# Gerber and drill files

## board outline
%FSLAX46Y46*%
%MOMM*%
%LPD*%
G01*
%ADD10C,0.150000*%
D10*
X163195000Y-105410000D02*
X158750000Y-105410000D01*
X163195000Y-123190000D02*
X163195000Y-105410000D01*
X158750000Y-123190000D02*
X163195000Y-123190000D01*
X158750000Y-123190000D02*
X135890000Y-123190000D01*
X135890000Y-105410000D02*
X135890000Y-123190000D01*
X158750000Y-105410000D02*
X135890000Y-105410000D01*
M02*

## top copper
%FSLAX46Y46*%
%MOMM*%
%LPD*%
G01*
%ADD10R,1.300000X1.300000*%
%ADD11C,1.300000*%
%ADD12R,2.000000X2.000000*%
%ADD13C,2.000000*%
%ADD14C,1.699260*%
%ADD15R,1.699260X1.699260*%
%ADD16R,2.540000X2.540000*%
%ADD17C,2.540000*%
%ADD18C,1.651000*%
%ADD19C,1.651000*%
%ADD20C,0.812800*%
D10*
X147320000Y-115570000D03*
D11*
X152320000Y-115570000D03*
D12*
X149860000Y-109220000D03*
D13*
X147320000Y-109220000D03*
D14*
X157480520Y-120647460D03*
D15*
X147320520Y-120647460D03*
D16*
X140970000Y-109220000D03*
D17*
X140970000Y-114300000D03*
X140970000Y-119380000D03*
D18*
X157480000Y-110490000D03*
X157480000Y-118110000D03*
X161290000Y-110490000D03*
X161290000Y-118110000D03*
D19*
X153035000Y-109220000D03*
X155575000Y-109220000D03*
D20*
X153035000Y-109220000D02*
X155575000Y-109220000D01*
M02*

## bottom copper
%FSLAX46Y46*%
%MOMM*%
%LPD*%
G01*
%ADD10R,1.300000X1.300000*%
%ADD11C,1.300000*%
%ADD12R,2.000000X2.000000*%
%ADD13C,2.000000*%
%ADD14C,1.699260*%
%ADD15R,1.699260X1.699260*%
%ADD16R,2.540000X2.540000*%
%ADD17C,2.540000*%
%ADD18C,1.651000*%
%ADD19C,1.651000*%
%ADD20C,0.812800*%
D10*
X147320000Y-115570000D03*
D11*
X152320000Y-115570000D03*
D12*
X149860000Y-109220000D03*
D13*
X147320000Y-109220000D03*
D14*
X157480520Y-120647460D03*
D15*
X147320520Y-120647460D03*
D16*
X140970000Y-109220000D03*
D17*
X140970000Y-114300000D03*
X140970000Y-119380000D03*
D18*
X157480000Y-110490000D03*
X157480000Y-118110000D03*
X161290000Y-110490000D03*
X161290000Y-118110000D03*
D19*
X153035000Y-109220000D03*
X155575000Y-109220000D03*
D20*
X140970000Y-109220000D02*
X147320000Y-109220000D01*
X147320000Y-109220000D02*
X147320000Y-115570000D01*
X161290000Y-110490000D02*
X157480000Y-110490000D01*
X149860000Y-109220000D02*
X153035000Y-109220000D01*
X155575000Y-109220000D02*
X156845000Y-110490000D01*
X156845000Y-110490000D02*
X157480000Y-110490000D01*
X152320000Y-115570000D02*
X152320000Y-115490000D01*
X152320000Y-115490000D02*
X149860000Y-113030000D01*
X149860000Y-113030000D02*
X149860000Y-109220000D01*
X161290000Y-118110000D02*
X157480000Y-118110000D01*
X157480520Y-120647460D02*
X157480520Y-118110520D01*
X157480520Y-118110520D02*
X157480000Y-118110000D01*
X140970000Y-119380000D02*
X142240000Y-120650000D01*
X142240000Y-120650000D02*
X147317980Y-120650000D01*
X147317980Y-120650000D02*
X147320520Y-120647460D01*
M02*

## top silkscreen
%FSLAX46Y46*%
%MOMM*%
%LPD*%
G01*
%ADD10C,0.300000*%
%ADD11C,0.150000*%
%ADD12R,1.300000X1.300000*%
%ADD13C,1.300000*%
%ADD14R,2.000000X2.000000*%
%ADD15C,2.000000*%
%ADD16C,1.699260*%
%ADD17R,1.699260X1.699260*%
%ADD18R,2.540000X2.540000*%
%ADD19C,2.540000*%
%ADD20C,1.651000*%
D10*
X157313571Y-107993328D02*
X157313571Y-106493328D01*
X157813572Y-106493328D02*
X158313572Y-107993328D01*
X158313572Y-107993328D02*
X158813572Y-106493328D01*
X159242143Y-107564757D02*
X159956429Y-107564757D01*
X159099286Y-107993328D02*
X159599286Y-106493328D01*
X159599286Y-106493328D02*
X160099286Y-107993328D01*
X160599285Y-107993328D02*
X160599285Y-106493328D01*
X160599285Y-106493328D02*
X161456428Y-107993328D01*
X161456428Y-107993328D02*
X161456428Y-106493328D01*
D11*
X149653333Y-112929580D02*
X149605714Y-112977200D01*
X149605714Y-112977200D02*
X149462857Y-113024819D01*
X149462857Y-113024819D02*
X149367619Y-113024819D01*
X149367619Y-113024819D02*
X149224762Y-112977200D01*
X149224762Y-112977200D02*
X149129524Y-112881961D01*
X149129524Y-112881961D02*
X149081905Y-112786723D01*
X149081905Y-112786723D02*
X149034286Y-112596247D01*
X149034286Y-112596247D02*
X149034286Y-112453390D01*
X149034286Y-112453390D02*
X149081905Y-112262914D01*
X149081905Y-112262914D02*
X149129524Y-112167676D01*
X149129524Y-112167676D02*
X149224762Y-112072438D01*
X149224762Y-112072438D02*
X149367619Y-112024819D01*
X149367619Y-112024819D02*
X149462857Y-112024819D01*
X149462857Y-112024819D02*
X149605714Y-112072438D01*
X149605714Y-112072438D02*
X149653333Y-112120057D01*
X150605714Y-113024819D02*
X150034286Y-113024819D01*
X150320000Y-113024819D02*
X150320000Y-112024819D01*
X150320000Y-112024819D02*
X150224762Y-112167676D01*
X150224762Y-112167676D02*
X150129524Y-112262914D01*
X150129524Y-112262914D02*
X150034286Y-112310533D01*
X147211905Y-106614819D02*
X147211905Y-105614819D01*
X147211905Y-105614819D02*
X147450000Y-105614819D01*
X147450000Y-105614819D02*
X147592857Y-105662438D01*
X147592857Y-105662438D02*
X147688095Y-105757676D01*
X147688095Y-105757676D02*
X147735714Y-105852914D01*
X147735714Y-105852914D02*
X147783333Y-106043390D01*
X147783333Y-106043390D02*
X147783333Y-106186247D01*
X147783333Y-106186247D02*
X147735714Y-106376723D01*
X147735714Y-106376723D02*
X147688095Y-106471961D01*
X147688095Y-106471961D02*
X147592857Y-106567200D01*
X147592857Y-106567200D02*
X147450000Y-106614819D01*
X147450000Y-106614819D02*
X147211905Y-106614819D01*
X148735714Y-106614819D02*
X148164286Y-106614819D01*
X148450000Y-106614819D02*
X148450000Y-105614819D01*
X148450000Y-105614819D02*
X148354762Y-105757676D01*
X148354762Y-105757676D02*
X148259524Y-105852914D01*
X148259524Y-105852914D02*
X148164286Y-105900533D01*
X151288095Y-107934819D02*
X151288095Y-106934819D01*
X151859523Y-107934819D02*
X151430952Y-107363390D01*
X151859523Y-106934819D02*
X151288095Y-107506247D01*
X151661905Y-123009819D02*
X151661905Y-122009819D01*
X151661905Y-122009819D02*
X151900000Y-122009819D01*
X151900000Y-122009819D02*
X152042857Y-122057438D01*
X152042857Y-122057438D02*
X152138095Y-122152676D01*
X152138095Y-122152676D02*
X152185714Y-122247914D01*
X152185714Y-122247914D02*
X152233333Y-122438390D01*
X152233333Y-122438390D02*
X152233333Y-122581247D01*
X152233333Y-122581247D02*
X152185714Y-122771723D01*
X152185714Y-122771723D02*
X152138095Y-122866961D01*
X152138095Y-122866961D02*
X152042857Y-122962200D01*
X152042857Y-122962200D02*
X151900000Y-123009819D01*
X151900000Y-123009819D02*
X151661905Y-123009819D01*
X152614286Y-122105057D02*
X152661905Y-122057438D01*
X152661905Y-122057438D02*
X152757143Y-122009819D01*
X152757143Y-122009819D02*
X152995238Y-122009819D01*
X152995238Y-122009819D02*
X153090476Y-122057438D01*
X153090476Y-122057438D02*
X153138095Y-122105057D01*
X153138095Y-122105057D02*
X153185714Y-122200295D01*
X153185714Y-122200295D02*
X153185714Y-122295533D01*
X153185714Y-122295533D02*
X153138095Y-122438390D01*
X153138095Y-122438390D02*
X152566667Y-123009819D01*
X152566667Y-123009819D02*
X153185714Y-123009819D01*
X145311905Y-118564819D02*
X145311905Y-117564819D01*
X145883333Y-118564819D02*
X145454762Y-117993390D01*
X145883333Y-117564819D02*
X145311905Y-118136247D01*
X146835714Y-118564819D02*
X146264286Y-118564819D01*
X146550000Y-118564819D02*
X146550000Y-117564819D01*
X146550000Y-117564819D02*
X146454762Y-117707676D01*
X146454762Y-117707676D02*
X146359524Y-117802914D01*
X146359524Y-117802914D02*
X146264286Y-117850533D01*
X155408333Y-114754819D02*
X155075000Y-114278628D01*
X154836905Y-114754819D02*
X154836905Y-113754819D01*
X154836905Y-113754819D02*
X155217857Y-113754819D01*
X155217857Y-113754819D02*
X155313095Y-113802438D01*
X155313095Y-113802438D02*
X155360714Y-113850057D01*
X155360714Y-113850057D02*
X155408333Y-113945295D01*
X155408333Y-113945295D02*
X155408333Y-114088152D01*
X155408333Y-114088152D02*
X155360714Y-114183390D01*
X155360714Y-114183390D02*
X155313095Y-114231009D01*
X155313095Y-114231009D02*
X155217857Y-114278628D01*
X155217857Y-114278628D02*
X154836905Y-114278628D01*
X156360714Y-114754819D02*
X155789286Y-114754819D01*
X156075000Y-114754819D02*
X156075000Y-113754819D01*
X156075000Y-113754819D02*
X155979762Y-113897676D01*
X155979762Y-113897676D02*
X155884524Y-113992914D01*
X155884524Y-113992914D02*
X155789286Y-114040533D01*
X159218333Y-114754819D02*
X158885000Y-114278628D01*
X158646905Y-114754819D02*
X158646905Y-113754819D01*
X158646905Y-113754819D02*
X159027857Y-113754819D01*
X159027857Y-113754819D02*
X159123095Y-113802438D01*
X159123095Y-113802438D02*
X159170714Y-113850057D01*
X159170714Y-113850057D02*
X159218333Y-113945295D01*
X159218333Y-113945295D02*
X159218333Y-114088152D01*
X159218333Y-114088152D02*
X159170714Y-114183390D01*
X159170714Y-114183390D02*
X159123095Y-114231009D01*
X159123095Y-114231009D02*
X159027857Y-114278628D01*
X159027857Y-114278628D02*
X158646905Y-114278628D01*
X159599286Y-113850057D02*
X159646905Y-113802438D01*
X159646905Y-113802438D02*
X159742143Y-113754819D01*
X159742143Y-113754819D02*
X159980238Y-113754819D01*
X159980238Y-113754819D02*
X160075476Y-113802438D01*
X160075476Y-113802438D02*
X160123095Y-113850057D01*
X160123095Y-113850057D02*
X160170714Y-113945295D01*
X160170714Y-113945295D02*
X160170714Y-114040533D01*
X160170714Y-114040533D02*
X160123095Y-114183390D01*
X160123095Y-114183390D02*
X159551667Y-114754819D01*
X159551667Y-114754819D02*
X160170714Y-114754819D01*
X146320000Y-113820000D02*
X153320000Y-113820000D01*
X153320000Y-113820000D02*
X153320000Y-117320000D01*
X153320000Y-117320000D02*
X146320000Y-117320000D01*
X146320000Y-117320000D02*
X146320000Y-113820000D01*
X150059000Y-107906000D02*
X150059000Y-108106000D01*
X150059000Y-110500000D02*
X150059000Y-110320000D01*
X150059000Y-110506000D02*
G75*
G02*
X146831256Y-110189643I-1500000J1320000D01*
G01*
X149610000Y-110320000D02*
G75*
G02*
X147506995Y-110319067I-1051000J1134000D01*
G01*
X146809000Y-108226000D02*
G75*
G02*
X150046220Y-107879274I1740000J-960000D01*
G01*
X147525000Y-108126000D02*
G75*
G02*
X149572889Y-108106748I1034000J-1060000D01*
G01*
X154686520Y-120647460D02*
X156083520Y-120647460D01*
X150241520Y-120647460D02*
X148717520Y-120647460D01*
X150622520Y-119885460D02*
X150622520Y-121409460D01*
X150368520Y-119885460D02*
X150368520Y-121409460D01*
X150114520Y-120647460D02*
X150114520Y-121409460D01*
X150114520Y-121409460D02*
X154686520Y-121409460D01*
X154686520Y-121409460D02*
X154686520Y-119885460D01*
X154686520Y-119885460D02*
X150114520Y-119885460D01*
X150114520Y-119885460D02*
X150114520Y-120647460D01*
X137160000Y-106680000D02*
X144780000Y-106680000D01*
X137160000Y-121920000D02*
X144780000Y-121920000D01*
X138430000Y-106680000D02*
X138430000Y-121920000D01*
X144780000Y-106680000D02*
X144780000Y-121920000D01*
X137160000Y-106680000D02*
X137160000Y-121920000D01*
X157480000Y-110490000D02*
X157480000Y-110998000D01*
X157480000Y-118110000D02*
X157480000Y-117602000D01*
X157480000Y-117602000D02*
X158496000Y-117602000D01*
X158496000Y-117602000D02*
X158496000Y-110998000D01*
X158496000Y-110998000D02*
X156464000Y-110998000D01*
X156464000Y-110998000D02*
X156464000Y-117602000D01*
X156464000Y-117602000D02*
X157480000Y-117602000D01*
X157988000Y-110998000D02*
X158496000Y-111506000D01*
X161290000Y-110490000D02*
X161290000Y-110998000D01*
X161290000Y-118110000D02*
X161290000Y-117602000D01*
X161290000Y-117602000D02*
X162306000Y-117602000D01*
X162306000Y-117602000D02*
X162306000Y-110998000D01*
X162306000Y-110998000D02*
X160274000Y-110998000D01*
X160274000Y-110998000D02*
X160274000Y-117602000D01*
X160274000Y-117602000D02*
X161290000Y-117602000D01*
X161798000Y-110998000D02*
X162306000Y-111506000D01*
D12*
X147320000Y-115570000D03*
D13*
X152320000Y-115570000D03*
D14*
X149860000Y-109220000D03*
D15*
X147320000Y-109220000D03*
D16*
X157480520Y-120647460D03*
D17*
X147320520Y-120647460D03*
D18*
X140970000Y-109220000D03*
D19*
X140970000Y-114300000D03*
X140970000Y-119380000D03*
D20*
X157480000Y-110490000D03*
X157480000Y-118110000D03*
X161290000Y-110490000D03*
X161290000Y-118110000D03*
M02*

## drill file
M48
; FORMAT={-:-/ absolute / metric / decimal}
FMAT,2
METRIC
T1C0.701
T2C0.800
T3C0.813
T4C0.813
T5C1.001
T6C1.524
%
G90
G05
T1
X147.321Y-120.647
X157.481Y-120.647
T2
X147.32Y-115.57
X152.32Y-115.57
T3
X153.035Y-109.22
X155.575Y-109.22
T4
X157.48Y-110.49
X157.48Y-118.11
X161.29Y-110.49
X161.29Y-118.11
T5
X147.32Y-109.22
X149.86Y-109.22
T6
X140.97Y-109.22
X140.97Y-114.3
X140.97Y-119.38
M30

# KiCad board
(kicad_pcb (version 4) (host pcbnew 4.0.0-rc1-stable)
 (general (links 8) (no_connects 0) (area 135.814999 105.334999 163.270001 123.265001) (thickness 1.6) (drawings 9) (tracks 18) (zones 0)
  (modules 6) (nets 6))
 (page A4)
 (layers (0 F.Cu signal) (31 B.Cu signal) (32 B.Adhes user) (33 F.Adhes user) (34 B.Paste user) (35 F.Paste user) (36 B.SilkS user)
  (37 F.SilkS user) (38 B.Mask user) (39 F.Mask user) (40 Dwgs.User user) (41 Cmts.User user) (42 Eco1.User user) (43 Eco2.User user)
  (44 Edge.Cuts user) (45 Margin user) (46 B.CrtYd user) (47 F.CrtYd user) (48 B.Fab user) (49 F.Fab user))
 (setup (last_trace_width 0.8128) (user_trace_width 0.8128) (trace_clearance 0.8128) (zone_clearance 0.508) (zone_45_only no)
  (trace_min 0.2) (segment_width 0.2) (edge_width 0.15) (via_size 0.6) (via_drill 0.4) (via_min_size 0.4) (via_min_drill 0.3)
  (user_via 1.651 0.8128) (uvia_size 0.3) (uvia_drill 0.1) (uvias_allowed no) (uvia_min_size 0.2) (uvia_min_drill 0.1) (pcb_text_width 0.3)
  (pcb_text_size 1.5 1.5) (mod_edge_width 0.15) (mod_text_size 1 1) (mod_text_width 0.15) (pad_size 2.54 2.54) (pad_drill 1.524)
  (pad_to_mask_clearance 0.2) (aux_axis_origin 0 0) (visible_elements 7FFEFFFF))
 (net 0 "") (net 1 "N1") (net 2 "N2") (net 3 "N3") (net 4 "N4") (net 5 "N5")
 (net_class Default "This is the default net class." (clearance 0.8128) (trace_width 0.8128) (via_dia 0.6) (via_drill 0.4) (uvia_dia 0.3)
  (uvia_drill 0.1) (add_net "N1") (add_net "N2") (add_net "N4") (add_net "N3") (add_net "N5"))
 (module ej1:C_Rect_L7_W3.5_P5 (layer F.Cu) (at 147.32 115.57)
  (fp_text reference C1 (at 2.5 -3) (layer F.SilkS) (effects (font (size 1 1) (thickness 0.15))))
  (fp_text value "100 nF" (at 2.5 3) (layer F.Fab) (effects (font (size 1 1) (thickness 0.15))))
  (fp_line (start -1 -1.75) (end 6 -1.75) (layer F.SilkS) (width 0.15))
  (fp_line (start 6 -1.75) (end 6 1.75) (layer F.SilkS) (width 0.15))
  (fp_line (start 6 1.75) (end -1 1.75) (layer F.SilkS) (width 0.15))
  (fp_line (start -1 1.75) (end -1 -1.75) (layer F.SilkS) (width 0.15))
  (pad 1 thru_hole rect (at 0 0) (size 1.3 1.3) (drill 0.8) (layers *.Cu *.Mask F.SilkS) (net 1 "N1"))
  (pad 2 thru_hole circle (at 5 0) (size 1.3 1.3) (drill 0.8) (layers *.Cu *.Mask F.SilkS) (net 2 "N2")))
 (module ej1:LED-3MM (layer F.Cu) (at 149.86 109.22 180)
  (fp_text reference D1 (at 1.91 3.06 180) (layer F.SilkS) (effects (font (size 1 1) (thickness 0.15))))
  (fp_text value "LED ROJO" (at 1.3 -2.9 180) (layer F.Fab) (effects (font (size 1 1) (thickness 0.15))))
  (fp_line (start -0.199 1.314) (end -0.199 1.114) (layer F.SilkS) (width 0.15))
  (fp_line (start -0.199 -1.28) (end -0.199 -1.1) (layer F.SilkS) (width 0.15))
  (fp_arc (start 1.301 0.034) (end -0.199 -1.286) (angle 108.5) (layer F.SilkS) (width 0.15))
  (fp_arc (start 1.301 0.034) (end 0.25 -1.1) (angle 85.7) (layer F.SilkS) (width 0.15))
  (fp_arc (start 1.311 0.034) (end 3.051 0.994) (angle 110) (layer F.SilkS) (width 0.15))
  (fp_arc (start 1.301 0.034) (end 2.335 1.094) (angle 87.5) (layer F.SilkS) (width 0.15))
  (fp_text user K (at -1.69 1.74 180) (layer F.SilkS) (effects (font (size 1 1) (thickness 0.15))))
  (pad 1 thru_hole rect (at 0 0 270) (size 2 2) (drill 1.00076) (layers *.Cu *.Mask F.SilkS) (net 2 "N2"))
  (pad 2 thru_hole circle (at 2.54 0 180) (size 2 2) (drill 1.00076) (layers *.Cu *.Mask F.SilkS) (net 1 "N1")))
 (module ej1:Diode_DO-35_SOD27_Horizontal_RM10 (layer F.Cu) (at 147.32 120.65)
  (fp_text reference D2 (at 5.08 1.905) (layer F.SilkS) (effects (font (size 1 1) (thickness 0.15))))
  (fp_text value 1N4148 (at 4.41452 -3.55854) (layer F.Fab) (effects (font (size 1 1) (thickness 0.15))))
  (fp_line (start 7.36652 -0.00254) (end 8.76352 -0.00254) (layer F.SilkS) (width 0.15))
  (fp_line (start 2.92152 -0.00254) (end 1.39752 -0.00254) (layer F.SilkS) (width 0.15))
  (fp_line (start 3.30252 -0.76454) (end 3.30252 0.75946) (layer F.SilkS) (width 0.15))
  (fp_line (start 3.04852 -0.76454) (end 3.04852 0.75946) (layer F.SilkS) (width 0.15))
  (fp_line (start 2.79452 -0.00254) (end 2.79452 0.75946) (layer F.SilkS) (width 0.15))
  (fp_line (start 2.79452 0.75946) (end 7.36652 0.75946) (layer F.SilkS) (width 0.15))
  (fp_line (start 7.36652 0.75946) (end 7.36652 -0.76454) (layer F.SilkS) (width 0.15))
  (fp_line (start 7.36652 -0.76454) (end 2.79452 -0.76454) (layer F.SilkS) (width 0.15))
  (fp_line (start 2.79452 -0.76454) (end 2.79452 -0.00254) (layer F.SilkS) (width 0.15))
  (pad 2 thru_hole circle (at 10.16052 -0.00254 180) (size 1.69926 1.69926) (drill 0.70104) (layers *.Cu *.Mask F.SilkS) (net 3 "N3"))
  (pad 1 thru_hole rect (at 0.00052 -0.00254 180) (size 1.69926 1.69926) (drill 0.70104) (layers *.Cu *.Mask F.SilkS) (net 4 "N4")))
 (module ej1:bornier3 (layer F.Cu) (at 140.97 114.3 270)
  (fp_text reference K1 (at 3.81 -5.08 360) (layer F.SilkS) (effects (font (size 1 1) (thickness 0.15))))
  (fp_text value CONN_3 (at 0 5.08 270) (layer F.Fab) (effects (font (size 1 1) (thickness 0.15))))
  (fp_line (start -7.62 3.81) (end -7.62 -3.81) (layer F.SilkS) (width 0.15))
  (fp_line (start 7.62 3.81) (end 7.62 -3.81) (layer F.SilkS) (width 0.15))
  (fp_line (start -7.62 2.54) (end 7.62 2.54) (layer F.SilkS) (width 0.15))
  (fp_line (start -7.62 -3.81) (end 7.62 -3.81) (layer F.SilkS) (width 0.15))
  (fp_line (start -7.62 3.81) (end 7.62 3.81) (layer F.SilkS) (width 0.15))
  (pad 1 thru_hole rect (at -5.08 0 270) (size 2.54 2.54) (drill 1.524) (layers *.Cu *.Mask F.SilkS) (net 1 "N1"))
  (pad 2 thru_hole circle (at 0 0 270) (size 2.54 2.54) (drill 1.524) (layers *.Cu *.Mask F.SilkS) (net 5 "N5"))
  (pad 3 thru_hole circle (at 5.08 0 270) (size 2.54 2.54) (drill 1.524) (layers *.Cu *.Mask F.SilkS) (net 4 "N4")))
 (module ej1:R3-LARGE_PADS (layer F.Cu) (at 157.48 114.3 270)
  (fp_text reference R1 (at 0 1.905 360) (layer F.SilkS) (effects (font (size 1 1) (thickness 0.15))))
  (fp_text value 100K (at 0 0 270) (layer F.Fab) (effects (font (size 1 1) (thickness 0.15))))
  (fp_line (start -3.81 0) (end -3.302 0) (layer F.SilkS) (width 0.15))
  (fp_line (start 3.81 0) (end 3.302 0) (layer F.SilkS) (width 0.15))
  (fp_line (start 3.302 0) (end 3.302 -1.016) (layer F.SilkS) (width 0.15))
  (fp_line (start 3.302 -1.016) (end -3.302 -1.016) (layer F.SilkS) (width 0.15))
  (fp_line (start -3.302 -1.016) (end -3.302 1.016) (layer F.SilkS) (width 0.15))
  (fp_line (start -3.302 1.016) (end 3.302 1.016) (layer F.SilkS) (width 0.15))
  (fp_line (start 3.302 1.016) (end 3.302 0) (layer F.SilkS) (width 0.15))
  (fp_line (start -3.302 -0.508) (end -2.794 -1.016) (layer F.SilkS) (width 0.15))
  (pad 1 thru_hole circle (at -3.81 0 270) (size 1.651 1.651) (drill 0.8128) (layers *.Cu *.Mask F.SilkS) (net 2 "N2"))
  (pad 2 thru_hole circle (at 3.81 0 270) (size 1.651 1.651) (drill 0.8128) (layers *.Cu *.Mask F.SilkS) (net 3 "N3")))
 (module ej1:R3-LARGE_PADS (layer F.Cu) (at 161.29 114.3 270)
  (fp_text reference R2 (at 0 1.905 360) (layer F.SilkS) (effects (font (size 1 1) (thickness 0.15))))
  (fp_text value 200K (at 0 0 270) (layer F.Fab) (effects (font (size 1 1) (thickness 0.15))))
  (fp_line (start -3.81 0) (end -3.302 0) (layer F.SilkS) (width 0.15))
  (fp_line (start 3.81 0) (end 3.302 0) (layer F.SilkS) (width 0.15))
  (fp_line (start 3.302 0) (end 3.302 -1.016) (layer F.SilkS) (width 0.15))
  (fp_line (start 3.302 -1.016) (end -3.302 -1.016) (layer F.SilkS) (width 0.15))
  (fp_line (start -3.302 -1.016) (end -3.302 1.016) (layer F.SilkS) (width 0.15))
  (fp_line (start -3.302 1.016) (end 3.302 1.016) (layer F.SilkS) (width 0.15))
  (fp_line (start 3.302 1.016) (end 3.302 0) (layer F.SilkS) (width 0.15))
  (fp_line (start -3.302 -0.508) (end -2.794 -1.016) (layer F.SilkS) (width 0.15))
  (pad 1 thru_hole circle (at -3.81 0 270) (size 1.651 1.651) (drill 0.8128) (layers *.Cu *.Mask F.SilkS) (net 2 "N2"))
  (pad 2 thru_hole circle (at 3.81 0 270) (size 1.651 1.651) (drill 0.8128) (layers *.Cu *.Mask F.SilkS) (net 3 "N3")))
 (gr_line (start 163.195 105.41) (end 158.75 105.41) (angle 90) (layer Edge.Cuts) (width 0.15))
 (gr_line (start 163.195 123.19) (end 163.195 105.41) (angle 90) (layer Edge.Cuts) (width 0.15))
 (gr_line (start 158.75 123.19) (end 163.195 123.19) (angle 90) (layer Edge.Cuts) (width 0.15))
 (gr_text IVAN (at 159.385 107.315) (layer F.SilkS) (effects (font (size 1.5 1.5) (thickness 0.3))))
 (gr_line (start 158.75 123.19) (end 135.89 123.19) (angle 90) (layer Edge.Cuts) (width 0.15))
 (gr_line (start 135.89 105.41) (end 135.89 123.19) (angle 90) (layer Edge.Cuts) (width 0.15))
 (gr_line (start 158.75 105.41) (end 135.89 105.41) (angle 90) (layer Edge.Cuts) (width 0.15))
 (segment (start 140.97 109.22) (end 147.32 109.22) (width 0.8128) (layer B.Cu) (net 1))
 (segment (start 147.32 109.22) (end 147.32 115.57) (width 0.8128) (layer B.Cu) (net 1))
 (segment (start 161.29 110.49) (end 157.48 110.49) (width 0.8128) (layer B.Cu) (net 2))
 (segment (start 149.86 109.22) (end 153.035 109.22) (width 0.8128) (layer B.Cu) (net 2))
 (via (at 153.035 109.22) (size 1.651) (drill 0.8128) (layers F.Cu B.Cu) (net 2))
 (segment (start 153.035 109.22) (end 155.575 109.22) (width 0.8128) (layer F.Cu) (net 2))
 (via (at 155.575 109.22) (size 1.651) (drill 0.8128) (layers F.Cu B.Cu) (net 2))
 (segment (start 155.575 109.22) (end 156.845 110.49) (width 0.8128) (layer B.Cu) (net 2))
 (segment (start 156.845 110.49) (end 157.48 110.49) (width 0.8128) (layer B.Cu) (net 2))
 (segment (start 152.32 115.57) (end 152.32 115.49) (width 0.8128) (layer B.Cu) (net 2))
 (segment (start 152.32 115.49) (end 149.86 113.03) (width 0.8128) (layer B.Cu) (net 2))
 (segment (start 149.86 113.03) (end 149.86 109.22) (width 0.8128) (layer B.Cu) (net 2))
 (segment (start 161.29 118.11) (end 157.48 118.11) (width 0.8128) (layer B.Cu) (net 3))
 (segment (start 157.48052 120.64746) (end 157.48052 118.11052) (width 0.8128) (layer B.Cu) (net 3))
 (segment (start 157.48052 118.11052) (end 157.48 118.11) (width 0.8128) (layer B.Cu) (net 3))
 (segment (start 140.97 119.38) (end 142.24 120.65) (width 0.8128) (layer B.Cu) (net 4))
 (segment (start 142.24 120.65) (end 147.31798 120.65) (width 0.8128) (layer B.Cu) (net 4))
 (segment (start 147.31798 120.65) (end 147.32052 120.64746) (width 0.8128) (layer B.Cu) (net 4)))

